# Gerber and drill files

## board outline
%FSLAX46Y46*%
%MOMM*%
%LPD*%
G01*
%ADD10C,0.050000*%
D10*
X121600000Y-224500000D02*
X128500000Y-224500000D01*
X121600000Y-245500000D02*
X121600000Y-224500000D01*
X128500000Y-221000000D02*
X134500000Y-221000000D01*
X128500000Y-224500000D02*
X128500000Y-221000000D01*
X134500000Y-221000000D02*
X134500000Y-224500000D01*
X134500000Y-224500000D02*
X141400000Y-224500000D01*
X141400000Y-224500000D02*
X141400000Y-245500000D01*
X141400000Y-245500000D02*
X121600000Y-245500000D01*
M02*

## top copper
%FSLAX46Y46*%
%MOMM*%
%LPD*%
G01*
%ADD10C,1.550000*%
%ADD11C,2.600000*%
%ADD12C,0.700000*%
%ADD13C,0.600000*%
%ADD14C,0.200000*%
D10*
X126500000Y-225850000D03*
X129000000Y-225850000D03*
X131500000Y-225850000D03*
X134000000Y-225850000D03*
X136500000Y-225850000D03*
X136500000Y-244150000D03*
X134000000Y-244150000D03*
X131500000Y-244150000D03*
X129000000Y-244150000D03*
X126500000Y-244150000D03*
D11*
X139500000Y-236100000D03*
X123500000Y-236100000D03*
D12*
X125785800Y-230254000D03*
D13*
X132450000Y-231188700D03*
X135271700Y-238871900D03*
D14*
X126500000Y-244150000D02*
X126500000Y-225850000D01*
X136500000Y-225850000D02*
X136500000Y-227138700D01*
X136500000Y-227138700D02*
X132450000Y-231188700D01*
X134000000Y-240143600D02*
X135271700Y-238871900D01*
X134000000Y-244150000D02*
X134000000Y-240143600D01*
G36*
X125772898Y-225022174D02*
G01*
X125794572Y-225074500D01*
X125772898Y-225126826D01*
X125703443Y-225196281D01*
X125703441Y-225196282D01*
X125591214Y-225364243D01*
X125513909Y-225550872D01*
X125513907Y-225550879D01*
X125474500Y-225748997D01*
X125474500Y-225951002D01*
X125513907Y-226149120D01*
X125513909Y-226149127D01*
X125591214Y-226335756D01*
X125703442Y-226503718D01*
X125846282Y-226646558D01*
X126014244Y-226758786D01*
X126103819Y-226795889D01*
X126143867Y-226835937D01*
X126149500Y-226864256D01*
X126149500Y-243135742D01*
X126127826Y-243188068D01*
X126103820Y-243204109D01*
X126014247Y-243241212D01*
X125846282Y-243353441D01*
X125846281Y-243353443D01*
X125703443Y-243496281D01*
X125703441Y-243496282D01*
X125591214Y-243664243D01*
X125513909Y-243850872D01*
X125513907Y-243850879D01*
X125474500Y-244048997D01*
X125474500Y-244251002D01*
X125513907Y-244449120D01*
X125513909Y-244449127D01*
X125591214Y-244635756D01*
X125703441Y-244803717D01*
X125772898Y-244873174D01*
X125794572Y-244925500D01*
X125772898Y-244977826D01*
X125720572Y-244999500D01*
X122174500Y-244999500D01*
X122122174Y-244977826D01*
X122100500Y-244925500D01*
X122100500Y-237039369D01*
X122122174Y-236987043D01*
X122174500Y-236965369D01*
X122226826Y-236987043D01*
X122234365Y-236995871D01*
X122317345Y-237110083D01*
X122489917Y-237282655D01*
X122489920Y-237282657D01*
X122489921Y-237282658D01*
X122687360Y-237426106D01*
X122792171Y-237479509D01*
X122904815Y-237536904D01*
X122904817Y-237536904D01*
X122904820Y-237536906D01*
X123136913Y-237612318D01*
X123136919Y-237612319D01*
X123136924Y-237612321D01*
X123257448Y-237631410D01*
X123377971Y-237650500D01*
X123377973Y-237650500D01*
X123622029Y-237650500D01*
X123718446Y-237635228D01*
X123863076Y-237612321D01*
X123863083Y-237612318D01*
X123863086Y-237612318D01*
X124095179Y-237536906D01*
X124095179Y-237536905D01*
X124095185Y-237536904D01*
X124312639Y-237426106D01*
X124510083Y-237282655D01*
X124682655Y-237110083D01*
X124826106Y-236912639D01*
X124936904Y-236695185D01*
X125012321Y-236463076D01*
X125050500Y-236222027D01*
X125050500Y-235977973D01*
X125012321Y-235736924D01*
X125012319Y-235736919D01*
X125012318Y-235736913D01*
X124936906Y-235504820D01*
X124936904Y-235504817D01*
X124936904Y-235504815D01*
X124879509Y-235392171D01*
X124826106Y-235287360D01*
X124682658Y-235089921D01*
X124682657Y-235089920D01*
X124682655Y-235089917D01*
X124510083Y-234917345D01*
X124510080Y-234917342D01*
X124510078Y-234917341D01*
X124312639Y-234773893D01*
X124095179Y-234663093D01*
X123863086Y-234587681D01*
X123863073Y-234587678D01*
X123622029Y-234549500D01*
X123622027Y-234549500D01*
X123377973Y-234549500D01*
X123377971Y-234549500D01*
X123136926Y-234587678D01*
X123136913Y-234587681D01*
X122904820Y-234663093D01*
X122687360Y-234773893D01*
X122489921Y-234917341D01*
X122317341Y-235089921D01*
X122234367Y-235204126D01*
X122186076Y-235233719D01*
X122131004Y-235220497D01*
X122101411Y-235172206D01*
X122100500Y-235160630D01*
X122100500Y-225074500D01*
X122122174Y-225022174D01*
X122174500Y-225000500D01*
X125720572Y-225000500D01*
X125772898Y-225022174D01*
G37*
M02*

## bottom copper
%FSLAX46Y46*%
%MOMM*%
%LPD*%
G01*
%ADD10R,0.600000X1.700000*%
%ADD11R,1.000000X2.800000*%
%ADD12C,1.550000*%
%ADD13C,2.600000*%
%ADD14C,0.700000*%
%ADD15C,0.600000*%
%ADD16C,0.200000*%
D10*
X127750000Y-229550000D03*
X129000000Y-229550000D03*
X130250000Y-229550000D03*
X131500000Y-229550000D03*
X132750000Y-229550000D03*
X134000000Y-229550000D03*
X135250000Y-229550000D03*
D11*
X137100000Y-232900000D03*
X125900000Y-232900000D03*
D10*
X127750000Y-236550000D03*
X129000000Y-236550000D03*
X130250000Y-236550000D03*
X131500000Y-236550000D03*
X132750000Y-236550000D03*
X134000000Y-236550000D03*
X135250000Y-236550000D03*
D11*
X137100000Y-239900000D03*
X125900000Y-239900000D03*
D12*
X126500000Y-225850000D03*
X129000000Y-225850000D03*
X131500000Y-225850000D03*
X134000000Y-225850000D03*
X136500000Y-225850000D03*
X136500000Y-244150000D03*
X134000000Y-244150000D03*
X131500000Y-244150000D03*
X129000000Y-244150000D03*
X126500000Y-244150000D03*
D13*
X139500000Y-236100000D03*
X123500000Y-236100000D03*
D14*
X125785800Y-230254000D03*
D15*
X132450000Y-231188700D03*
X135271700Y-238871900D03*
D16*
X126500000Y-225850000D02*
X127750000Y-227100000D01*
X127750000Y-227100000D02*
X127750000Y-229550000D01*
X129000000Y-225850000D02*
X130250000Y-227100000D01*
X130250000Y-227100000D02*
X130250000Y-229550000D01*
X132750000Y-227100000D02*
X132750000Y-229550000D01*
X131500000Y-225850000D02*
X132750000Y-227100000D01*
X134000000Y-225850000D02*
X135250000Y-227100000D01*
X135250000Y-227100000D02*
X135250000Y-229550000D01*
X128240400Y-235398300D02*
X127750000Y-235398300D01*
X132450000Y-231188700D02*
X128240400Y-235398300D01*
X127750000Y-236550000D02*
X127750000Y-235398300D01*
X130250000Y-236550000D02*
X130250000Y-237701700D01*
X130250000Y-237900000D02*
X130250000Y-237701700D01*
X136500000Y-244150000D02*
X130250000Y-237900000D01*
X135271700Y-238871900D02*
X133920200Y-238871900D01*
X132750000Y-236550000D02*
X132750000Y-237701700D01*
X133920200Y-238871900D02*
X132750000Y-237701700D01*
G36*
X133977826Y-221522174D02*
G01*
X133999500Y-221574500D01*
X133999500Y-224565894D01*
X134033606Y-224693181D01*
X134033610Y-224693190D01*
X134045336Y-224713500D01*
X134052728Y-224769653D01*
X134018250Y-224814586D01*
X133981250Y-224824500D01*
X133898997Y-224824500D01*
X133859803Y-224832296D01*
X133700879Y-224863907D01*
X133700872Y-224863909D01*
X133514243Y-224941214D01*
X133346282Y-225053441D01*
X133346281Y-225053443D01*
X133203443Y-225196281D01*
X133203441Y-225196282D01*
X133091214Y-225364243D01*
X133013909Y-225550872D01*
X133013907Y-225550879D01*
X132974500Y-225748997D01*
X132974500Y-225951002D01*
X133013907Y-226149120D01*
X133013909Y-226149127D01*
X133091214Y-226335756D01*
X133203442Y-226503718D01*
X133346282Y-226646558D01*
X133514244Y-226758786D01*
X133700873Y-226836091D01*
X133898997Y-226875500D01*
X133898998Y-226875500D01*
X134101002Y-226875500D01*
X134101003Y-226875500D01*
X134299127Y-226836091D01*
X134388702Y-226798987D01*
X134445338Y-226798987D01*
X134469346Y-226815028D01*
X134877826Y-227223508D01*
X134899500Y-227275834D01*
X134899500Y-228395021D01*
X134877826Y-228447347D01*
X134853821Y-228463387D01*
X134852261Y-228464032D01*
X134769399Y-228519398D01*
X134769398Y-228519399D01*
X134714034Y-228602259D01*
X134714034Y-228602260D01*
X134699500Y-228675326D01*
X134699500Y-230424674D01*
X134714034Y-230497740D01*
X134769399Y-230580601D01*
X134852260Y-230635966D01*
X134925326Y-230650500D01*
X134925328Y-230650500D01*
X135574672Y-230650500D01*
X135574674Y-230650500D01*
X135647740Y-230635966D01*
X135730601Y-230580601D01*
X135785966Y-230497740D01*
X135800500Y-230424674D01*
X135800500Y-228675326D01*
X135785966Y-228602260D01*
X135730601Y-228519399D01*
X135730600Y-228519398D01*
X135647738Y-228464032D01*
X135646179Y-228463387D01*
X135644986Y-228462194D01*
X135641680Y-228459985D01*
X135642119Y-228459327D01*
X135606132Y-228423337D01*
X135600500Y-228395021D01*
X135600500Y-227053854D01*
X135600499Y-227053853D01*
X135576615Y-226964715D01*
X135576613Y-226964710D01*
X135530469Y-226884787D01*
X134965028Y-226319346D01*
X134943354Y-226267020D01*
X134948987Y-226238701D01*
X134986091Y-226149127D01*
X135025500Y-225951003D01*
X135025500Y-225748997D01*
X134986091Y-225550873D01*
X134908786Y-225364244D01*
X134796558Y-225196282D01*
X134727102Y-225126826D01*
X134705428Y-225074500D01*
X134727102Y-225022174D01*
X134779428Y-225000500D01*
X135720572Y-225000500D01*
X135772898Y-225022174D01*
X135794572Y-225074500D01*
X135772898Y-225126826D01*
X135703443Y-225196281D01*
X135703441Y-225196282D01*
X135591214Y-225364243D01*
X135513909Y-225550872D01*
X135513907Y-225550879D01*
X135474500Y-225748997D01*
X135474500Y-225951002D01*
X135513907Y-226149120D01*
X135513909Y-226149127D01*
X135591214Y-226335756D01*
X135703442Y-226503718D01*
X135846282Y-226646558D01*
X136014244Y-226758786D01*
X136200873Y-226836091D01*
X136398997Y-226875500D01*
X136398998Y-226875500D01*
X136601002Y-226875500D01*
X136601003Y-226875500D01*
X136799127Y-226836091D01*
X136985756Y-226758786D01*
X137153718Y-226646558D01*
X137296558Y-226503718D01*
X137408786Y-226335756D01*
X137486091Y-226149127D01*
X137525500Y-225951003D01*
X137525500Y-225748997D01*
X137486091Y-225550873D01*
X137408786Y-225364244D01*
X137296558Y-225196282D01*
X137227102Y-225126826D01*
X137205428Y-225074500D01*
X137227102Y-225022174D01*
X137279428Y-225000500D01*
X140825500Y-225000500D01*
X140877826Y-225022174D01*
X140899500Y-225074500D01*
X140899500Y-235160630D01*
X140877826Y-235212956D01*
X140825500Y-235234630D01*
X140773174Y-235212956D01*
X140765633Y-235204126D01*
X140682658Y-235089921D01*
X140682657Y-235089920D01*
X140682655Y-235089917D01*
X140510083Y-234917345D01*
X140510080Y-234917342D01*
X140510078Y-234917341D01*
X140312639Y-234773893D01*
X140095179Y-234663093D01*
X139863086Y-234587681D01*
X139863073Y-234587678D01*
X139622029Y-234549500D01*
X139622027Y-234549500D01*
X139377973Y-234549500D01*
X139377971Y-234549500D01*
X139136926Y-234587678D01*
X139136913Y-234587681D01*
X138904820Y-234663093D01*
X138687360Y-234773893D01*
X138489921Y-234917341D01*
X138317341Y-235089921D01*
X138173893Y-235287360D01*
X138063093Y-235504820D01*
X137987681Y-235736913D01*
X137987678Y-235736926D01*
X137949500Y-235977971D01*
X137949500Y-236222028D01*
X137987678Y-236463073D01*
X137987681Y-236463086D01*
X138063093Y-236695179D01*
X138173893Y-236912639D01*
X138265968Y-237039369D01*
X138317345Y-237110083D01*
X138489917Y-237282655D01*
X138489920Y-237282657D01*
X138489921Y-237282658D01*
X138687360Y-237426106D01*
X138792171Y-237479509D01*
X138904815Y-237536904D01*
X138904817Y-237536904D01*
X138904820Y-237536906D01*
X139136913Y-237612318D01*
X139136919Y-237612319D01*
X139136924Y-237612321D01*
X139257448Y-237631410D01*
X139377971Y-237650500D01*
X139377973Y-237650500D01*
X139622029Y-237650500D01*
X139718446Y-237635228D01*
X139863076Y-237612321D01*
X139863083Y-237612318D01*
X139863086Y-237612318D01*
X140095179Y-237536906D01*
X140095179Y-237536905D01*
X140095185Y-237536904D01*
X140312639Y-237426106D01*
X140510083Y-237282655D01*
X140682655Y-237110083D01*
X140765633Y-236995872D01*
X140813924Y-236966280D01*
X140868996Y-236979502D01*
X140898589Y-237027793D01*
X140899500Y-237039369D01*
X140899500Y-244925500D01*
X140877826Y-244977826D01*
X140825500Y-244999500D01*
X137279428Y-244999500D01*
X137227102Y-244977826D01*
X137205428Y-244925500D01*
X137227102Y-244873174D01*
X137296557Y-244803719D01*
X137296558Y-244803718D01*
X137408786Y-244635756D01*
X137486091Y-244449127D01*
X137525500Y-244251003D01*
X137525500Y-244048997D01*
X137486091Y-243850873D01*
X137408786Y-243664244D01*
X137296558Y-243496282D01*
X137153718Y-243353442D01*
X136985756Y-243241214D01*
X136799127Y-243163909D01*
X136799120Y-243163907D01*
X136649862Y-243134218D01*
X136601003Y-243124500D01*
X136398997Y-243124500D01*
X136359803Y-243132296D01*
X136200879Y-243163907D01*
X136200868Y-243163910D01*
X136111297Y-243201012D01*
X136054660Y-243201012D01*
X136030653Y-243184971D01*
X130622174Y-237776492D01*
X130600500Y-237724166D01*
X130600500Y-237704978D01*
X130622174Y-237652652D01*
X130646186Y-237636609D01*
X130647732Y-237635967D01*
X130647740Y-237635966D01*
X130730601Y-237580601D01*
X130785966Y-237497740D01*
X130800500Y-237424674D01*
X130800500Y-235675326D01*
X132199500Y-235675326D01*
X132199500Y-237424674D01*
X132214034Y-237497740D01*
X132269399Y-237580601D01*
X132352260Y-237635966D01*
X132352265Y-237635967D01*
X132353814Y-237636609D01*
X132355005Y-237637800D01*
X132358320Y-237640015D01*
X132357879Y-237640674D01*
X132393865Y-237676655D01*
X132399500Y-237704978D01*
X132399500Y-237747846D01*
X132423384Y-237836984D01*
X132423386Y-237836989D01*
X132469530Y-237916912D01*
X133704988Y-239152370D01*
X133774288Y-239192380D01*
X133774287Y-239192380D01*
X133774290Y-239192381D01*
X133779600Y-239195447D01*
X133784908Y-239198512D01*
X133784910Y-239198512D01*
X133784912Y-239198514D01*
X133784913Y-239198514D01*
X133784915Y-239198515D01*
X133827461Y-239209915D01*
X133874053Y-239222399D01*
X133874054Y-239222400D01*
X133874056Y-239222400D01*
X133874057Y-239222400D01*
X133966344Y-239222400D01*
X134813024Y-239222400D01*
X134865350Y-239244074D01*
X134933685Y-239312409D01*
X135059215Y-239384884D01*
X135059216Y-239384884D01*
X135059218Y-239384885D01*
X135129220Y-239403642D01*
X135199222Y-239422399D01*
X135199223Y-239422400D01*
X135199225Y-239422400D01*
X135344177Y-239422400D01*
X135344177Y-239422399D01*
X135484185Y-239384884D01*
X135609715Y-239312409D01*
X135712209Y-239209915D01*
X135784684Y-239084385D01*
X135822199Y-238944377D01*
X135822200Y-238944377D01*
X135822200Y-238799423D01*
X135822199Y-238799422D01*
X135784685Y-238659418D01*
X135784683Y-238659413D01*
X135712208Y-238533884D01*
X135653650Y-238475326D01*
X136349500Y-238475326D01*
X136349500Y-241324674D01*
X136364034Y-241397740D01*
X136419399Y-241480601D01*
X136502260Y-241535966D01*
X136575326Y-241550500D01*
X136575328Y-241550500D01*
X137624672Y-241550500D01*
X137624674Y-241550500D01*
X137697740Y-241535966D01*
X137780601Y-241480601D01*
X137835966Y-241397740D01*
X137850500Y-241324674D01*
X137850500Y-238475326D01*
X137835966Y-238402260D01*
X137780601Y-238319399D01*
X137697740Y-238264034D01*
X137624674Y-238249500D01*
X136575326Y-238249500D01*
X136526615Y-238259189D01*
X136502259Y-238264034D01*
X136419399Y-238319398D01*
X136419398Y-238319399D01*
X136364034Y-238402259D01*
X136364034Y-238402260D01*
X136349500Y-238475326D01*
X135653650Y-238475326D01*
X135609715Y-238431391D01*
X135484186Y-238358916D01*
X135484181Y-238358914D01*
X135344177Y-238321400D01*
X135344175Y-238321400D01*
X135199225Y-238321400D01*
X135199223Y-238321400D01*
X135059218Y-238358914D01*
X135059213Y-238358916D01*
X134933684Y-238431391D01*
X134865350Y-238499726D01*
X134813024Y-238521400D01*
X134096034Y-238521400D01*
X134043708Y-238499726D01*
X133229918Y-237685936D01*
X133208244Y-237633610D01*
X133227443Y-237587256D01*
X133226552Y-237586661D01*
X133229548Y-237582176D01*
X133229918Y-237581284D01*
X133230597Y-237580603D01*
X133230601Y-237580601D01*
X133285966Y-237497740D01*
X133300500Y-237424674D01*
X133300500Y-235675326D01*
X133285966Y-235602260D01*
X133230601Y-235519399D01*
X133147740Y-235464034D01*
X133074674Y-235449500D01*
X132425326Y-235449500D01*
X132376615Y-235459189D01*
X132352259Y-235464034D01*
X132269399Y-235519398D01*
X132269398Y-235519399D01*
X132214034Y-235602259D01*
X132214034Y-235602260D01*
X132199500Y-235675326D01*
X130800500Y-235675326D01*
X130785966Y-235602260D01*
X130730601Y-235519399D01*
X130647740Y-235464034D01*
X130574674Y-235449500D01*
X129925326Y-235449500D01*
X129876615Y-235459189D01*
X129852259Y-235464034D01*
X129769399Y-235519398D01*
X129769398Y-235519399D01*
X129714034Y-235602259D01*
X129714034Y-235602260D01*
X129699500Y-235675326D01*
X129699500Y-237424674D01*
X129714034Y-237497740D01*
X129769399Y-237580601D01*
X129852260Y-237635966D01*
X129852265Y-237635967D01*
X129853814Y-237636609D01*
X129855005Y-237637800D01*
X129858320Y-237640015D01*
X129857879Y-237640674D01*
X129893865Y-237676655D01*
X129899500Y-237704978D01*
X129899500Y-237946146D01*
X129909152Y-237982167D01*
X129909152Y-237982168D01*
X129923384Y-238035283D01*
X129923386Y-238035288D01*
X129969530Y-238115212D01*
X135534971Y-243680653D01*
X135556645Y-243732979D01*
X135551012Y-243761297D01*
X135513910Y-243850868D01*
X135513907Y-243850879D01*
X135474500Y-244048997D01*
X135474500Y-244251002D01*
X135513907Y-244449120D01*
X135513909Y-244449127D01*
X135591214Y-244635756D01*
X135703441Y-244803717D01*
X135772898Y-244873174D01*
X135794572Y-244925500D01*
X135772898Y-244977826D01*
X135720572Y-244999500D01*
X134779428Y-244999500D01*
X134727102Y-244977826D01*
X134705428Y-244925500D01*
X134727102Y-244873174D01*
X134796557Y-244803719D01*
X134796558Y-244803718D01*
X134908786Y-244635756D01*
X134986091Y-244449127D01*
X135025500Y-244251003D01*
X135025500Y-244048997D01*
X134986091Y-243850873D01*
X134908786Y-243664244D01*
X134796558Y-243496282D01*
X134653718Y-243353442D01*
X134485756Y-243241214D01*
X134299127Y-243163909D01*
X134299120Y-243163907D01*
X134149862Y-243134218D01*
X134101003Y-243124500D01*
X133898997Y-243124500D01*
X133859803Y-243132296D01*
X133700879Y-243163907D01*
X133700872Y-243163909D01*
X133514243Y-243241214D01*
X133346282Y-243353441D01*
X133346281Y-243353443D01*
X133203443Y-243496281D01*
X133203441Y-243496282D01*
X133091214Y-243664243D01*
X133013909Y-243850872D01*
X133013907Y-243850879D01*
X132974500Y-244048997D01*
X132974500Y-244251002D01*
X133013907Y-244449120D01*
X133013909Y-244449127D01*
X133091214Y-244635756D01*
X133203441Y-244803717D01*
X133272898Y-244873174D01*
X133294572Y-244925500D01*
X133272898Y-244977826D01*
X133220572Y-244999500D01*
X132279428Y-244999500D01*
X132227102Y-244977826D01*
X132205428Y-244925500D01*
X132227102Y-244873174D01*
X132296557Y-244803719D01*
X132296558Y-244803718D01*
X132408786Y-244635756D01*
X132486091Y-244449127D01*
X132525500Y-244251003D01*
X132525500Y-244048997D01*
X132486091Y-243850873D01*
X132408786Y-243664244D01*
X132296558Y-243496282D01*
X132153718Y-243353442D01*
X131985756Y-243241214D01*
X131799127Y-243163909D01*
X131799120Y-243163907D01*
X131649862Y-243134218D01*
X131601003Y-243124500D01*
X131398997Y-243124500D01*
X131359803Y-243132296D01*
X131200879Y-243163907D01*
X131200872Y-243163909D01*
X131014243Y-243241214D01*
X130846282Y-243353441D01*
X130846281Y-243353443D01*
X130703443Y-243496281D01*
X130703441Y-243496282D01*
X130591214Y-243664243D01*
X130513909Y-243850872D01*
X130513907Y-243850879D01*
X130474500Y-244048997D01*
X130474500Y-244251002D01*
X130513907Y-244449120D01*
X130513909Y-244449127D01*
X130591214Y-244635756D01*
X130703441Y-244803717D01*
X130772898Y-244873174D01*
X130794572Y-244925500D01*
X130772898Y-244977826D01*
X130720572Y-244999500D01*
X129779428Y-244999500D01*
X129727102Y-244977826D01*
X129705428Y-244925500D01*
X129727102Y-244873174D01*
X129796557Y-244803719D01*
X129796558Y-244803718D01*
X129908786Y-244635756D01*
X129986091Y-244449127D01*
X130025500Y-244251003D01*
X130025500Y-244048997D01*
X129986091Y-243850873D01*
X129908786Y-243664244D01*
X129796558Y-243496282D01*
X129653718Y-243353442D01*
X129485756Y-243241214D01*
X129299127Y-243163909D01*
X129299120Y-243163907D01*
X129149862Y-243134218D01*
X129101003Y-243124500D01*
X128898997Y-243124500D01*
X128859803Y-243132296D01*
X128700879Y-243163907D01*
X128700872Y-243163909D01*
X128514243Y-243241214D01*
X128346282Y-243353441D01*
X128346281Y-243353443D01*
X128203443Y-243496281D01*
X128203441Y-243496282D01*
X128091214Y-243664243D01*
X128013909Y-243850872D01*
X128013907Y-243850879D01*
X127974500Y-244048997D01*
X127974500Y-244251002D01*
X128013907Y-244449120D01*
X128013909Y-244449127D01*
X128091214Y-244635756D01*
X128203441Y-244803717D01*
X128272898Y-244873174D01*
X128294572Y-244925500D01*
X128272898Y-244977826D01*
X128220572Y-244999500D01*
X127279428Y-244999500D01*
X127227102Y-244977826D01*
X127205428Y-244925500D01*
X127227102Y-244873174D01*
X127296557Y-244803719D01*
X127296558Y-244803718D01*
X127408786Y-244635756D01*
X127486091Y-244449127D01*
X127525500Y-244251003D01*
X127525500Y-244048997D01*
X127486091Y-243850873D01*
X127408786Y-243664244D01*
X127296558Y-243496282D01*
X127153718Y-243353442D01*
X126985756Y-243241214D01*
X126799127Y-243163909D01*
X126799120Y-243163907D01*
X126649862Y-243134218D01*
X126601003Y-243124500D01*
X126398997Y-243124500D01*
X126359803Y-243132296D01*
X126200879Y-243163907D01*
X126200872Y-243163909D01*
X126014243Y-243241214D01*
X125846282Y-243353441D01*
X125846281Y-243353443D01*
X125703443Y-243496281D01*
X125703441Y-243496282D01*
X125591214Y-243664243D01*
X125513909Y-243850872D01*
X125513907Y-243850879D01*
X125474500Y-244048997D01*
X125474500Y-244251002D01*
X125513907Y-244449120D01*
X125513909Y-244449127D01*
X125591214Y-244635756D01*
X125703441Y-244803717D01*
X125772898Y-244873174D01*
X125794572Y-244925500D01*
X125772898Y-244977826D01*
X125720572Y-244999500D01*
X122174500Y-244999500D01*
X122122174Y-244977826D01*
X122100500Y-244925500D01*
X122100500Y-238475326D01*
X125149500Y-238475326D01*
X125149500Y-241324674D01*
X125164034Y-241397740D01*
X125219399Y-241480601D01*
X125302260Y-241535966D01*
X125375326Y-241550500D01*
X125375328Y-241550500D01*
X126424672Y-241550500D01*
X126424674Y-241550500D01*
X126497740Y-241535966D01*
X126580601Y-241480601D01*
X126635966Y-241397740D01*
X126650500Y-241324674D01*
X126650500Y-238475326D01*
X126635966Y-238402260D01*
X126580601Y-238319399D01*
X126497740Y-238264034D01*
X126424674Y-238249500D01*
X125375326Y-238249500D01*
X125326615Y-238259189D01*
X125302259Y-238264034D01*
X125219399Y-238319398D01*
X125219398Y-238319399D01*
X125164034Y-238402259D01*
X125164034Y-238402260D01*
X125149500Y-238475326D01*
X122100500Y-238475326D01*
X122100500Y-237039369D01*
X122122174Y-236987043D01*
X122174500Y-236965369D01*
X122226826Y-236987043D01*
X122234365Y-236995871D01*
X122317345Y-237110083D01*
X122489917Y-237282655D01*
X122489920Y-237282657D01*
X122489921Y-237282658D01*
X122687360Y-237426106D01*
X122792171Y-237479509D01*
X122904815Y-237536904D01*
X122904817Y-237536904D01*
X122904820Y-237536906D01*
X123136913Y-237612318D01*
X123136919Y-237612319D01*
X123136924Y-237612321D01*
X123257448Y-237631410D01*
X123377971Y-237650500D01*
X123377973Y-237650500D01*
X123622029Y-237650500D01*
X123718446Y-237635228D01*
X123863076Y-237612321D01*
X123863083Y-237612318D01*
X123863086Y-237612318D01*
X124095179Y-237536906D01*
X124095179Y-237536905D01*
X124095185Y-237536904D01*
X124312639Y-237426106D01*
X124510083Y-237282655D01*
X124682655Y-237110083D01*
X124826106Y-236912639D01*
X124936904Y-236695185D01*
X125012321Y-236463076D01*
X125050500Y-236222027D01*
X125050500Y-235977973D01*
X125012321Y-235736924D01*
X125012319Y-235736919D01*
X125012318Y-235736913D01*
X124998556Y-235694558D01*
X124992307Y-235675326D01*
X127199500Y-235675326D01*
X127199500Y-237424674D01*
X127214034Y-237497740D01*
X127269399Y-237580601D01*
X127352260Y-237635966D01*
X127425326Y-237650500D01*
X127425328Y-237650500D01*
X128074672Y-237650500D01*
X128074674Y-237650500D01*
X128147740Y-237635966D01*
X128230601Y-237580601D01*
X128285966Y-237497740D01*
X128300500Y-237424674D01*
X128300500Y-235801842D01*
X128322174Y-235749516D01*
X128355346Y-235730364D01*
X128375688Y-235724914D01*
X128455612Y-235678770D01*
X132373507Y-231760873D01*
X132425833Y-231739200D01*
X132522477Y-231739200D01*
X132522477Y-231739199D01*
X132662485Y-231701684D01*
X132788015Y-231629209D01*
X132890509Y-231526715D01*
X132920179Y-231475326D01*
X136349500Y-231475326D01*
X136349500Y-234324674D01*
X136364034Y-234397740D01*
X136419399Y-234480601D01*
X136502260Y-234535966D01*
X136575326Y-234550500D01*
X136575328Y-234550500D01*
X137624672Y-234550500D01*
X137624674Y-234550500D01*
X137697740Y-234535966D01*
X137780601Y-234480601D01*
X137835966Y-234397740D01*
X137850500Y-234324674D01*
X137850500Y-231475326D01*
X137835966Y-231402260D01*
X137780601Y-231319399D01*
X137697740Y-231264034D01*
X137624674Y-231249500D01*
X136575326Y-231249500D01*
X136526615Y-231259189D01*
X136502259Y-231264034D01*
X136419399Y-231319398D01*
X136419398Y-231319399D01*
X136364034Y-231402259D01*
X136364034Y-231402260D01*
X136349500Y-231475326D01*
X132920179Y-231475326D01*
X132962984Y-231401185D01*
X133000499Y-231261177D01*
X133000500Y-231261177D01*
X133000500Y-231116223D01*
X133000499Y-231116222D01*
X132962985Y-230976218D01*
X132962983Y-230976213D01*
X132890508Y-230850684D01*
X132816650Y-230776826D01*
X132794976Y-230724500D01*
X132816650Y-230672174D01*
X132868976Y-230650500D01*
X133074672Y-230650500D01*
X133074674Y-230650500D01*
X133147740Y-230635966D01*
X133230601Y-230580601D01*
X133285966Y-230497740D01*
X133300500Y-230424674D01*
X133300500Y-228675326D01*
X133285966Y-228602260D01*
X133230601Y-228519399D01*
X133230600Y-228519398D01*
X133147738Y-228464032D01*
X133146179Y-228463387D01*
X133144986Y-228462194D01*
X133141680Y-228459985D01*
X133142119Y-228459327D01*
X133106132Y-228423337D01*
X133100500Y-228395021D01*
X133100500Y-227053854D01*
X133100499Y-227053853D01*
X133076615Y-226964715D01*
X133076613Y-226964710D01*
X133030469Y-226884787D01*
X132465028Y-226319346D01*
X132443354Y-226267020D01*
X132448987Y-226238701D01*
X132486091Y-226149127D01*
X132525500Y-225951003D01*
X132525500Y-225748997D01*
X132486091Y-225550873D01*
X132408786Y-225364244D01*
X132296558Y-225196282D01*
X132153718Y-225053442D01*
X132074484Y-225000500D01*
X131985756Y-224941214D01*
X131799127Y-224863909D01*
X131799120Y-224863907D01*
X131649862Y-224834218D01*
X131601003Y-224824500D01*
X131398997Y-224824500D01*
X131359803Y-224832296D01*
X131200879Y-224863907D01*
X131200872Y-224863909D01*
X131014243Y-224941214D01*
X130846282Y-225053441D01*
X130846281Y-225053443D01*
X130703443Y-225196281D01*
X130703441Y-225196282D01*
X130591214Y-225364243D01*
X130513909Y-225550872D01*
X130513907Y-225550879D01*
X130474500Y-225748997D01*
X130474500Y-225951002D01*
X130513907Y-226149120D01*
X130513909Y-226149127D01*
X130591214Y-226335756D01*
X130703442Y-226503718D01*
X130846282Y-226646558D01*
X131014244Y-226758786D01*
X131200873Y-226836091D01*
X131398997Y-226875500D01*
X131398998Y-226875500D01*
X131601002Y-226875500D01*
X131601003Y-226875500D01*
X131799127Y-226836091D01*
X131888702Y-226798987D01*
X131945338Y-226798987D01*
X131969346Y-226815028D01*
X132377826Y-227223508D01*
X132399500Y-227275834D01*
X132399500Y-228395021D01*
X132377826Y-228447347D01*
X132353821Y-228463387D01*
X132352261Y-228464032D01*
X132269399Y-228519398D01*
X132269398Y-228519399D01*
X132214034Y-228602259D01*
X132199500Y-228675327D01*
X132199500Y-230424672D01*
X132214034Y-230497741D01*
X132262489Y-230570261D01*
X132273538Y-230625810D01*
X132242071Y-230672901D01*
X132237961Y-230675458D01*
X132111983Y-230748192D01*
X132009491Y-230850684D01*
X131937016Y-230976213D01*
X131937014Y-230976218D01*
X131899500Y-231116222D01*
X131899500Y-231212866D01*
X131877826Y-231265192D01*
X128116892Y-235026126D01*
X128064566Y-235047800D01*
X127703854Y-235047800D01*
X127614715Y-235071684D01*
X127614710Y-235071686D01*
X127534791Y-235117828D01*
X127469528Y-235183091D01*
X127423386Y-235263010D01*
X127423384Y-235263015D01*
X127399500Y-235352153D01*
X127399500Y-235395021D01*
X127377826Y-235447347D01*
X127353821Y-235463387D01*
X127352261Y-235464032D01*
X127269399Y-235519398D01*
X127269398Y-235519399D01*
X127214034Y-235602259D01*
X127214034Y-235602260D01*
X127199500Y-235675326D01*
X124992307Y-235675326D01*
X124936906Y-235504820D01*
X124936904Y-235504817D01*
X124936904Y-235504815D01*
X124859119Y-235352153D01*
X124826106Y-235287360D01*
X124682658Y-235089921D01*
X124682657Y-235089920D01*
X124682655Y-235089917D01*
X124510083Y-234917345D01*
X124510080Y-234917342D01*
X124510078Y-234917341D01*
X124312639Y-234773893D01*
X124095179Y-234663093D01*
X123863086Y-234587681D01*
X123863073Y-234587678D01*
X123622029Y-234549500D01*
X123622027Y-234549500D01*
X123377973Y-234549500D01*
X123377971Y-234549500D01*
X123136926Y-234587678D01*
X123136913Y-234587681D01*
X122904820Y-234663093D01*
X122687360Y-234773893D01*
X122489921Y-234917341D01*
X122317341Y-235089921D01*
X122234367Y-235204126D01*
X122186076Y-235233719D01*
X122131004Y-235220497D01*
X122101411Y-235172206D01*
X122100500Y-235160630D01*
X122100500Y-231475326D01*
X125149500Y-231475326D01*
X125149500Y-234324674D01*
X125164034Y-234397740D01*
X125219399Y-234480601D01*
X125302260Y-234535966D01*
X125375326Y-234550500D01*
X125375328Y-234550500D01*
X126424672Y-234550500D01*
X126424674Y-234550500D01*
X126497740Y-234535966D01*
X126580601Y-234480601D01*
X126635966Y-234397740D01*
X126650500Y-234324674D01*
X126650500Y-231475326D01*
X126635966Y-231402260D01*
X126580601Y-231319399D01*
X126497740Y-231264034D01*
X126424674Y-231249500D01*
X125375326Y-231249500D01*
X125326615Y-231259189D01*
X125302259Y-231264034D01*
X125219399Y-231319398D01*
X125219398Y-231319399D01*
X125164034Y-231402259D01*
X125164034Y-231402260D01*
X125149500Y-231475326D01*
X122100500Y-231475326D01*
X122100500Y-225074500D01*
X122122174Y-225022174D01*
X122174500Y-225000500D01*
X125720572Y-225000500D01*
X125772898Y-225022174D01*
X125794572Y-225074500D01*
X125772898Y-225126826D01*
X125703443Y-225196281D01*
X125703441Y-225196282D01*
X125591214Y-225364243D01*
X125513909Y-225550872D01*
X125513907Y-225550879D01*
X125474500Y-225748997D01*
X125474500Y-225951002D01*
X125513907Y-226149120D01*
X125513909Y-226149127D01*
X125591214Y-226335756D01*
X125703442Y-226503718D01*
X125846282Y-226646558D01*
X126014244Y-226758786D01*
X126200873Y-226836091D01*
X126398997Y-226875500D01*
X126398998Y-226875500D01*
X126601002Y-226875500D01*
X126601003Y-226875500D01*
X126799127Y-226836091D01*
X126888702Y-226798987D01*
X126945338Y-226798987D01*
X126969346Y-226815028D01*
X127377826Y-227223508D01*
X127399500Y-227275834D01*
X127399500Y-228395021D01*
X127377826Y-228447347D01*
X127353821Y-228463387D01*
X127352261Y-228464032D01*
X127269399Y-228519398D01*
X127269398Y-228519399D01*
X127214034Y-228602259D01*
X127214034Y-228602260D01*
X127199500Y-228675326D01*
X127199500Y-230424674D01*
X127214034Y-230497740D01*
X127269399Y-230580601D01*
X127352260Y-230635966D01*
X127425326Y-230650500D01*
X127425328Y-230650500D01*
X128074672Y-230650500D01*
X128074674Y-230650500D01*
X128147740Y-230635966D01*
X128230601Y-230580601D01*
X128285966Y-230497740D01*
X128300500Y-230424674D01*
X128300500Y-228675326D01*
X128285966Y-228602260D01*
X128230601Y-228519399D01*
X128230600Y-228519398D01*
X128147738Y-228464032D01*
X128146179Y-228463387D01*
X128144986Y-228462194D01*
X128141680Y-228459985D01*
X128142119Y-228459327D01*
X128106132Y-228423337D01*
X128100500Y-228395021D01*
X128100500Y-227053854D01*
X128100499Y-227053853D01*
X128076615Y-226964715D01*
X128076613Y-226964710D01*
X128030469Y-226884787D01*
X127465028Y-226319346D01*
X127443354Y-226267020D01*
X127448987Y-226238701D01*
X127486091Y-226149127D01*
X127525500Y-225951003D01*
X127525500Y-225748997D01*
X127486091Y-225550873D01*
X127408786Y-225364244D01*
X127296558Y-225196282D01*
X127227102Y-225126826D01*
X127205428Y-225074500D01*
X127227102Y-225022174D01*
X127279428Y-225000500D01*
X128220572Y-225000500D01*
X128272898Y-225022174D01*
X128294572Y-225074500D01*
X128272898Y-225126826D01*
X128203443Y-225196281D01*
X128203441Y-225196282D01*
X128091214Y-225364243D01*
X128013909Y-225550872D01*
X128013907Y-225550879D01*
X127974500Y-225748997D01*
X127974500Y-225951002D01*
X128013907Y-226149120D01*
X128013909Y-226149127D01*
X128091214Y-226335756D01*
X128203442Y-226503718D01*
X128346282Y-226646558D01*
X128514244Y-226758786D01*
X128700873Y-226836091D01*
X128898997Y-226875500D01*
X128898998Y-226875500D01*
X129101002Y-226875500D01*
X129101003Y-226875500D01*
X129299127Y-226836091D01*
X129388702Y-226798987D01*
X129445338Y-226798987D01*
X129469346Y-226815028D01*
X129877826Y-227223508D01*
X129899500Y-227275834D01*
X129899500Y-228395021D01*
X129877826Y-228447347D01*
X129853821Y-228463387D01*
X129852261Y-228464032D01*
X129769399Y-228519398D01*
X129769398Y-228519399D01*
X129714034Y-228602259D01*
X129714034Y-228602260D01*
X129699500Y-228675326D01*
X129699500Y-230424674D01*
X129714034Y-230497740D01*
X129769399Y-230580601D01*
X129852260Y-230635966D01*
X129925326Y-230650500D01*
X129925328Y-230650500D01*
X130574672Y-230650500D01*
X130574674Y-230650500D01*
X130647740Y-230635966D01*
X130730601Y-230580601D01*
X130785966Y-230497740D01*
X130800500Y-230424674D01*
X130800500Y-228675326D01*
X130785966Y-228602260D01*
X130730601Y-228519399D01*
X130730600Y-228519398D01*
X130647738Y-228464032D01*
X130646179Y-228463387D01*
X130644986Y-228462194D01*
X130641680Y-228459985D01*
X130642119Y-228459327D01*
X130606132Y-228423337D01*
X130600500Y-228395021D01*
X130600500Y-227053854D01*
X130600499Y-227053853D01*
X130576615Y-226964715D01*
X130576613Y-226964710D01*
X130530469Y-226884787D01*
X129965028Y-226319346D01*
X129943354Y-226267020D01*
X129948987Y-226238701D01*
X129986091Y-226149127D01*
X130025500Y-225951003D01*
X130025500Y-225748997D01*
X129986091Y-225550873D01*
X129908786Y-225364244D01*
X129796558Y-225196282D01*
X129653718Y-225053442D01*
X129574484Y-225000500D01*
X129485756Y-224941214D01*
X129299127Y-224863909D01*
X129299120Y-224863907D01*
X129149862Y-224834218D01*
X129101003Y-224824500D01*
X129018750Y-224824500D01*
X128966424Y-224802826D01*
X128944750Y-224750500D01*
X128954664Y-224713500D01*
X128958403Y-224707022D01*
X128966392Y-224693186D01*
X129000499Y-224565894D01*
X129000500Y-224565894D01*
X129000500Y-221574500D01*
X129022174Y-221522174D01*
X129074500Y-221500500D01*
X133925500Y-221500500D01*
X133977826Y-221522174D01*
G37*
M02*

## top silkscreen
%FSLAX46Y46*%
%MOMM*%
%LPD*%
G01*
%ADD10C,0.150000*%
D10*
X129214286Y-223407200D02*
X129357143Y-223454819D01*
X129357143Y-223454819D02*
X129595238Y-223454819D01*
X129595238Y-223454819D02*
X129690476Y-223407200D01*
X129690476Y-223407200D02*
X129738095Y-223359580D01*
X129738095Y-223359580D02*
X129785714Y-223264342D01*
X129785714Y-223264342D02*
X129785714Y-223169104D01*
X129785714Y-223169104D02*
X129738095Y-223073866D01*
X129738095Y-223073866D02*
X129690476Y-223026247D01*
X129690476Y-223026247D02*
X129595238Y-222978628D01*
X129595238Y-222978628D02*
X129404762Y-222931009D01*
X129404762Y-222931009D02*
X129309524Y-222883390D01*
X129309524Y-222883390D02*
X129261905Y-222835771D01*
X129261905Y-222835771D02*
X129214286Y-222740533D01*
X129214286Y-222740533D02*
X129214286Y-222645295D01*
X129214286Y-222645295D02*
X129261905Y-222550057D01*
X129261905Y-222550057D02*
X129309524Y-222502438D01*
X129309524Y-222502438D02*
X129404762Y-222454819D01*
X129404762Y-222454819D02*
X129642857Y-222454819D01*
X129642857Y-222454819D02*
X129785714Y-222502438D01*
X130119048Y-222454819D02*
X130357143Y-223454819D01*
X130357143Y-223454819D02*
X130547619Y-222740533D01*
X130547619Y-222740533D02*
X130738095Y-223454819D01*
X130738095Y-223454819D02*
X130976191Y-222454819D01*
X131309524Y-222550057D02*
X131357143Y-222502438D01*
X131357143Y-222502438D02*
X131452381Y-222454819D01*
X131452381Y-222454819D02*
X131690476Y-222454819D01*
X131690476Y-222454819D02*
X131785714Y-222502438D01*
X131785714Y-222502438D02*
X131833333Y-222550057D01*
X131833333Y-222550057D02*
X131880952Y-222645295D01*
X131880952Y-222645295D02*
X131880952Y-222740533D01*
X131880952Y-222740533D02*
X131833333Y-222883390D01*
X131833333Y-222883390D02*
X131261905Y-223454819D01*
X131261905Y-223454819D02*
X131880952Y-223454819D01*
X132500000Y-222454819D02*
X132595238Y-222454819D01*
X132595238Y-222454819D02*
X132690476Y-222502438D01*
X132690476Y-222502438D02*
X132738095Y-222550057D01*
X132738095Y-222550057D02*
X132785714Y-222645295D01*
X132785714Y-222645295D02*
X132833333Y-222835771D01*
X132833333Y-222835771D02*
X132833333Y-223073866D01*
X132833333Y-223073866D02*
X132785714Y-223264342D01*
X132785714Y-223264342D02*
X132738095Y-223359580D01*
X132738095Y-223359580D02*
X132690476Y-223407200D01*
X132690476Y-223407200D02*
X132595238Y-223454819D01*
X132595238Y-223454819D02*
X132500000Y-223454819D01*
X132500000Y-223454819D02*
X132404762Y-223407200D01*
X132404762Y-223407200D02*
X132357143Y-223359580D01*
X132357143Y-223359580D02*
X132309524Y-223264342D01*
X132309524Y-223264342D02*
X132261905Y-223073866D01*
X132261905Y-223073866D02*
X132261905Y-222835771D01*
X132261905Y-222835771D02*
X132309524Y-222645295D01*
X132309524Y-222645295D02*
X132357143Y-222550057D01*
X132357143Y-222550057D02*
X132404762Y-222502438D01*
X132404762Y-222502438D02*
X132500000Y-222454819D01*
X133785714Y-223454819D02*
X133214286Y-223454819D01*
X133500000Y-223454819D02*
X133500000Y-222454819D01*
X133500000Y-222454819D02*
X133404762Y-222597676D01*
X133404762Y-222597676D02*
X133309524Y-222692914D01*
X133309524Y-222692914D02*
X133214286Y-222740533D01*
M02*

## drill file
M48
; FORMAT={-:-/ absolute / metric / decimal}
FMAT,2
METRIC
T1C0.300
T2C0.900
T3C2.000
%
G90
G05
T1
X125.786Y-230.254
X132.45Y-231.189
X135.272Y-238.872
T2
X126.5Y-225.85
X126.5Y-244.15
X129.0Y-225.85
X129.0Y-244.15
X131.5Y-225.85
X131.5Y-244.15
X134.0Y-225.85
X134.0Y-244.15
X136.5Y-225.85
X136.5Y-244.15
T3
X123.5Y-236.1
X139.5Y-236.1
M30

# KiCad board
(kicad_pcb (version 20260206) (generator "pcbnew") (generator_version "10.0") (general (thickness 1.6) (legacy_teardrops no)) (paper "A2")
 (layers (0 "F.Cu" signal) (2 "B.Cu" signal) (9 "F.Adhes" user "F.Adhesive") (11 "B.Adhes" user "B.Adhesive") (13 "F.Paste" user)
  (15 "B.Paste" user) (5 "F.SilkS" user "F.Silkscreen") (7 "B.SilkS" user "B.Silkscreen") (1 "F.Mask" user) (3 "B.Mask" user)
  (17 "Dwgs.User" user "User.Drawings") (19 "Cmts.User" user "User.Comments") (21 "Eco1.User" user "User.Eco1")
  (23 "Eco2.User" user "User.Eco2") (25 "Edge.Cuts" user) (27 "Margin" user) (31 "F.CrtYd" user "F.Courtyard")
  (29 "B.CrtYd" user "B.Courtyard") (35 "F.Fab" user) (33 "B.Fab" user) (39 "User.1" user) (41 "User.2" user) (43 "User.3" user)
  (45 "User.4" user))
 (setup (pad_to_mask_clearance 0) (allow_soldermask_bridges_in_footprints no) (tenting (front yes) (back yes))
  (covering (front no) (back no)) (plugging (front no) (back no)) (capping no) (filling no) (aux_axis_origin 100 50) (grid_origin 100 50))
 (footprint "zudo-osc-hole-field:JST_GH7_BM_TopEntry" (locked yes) (layer "B.Cu") (at 131.5 229.55 180)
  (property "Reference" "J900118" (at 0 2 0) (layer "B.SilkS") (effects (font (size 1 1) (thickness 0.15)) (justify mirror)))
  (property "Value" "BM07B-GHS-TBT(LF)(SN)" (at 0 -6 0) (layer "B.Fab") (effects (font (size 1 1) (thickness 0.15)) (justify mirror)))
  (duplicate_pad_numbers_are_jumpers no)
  (pad "1" smd rect (at 3.75 0 180) (size 0.6 1.7) (layers "B.Cu" "B.Mask" "B.Paste") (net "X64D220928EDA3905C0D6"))
  (pad "2" smd rect (at 2.5 0 180) (size 0.6 1.7) (layers "B.Cu" "B.Mask" "B.Paste") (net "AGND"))
  (pad "3" smd rect (at 1.25 0 180) (size 0.6 1.7) (layers "B.Cu" "B.Mask" "B.Paste") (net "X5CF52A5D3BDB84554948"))
  (pad "4" smd rect (at 0 0 180) (size 0.6 1.7) (layers "B.Cu" "B.Mask" "B.Paste") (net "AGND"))
  (pad "5" smd rect (at -1.25 0 180) (size 0.6 1.7) (layers "B.Cu" "B.Mask" "B.Paste") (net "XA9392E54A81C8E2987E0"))
  (pad "6" smd rect (at -2.5 0 180) (size 0.6 1.7) (layers "B.Cu" "B.Mask" "B.Paste") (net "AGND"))
  (pad "7" smd rect (at -3.75 0 180) (size 0.6 1.7) (layers "B.Cu" "B.Mask" "B.Paste") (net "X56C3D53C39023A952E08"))
  (pad "MP1" smd rect (at -5.6 -3.35 180) (size 1 2.8) (layers "B.Cu" "B.Mask" "B.Paste") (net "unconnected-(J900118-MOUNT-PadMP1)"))
  (pad "MP2" smd rect (at 5.6 -3.35 180) (size 1 2.8) (layers "B.Cu" "B.Mask" "B.Paste") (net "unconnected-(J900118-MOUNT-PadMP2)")))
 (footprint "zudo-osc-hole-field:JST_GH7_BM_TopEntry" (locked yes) (layer "B.Cu") (at 131.5 236.55 180)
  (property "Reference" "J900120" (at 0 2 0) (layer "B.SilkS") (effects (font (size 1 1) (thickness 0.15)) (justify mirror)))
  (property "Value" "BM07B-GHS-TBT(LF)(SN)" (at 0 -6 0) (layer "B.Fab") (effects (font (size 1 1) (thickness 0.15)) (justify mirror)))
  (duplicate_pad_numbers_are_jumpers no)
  (pad "1" smd rect (at 3.75 0 180) (size 0.6 1.7) (layers "B.Cu" "B.Mask" "B.Paste") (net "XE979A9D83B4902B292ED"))
  (pad "2" smd rect (at 2.5 0 180) (size 0.6 1.7) (layers "B.Cu" "B.Mask" "B.Paste") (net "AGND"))
  (pad "3" smd rect (at 1.25 0 180) (size 0.6 1.7) (layers "B.Cu" "B.Mask" "B.Paste") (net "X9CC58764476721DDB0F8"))
  (pad "4" smd rect (at 0 0 180) (size 0.6 1.7) (layers "B.Cu" "B.Mask" "B.Paste") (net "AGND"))
  (pad "5" smd rect (at -1.25 0 180) (size 0.6 1.7) (layers "B.Cu" "B.Mask" "B.Paste") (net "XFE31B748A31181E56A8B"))
  (pad "6" smd rect (at -2.5 0 180) (size 0.6 1.7) (layers "B.Cu" "B.Mask" "B.Paste") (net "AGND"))
  (pad "7" smd rect (at -3.75 0 180) (size 0.6 1.7) (layers "B.Cu" "B.Mask" "B.Paste") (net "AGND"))
  (pad "MP1" smd rect (at -5.6 -3.35 180) (size 1 2.8) (layers "B.Cu" "B.Mask" "B.Paste") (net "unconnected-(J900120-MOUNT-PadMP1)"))
  (pad "MP2" smd rect (at 5.6 -3.35 180) (size 1 2.8) (layers "B.Cu" "B.Mask" "B.Paste") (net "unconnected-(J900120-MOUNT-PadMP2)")))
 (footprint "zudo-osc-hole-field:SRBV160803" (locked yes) (layer "F.Cu") (at 131.5 235 180)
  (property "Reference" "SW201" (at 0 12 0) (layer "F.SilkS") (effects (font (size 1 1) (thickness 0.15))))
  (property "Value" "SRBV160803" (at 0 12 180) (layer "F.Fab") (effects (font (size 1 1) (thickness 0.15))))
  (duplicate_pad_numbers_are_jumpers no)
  (pad "1" thru_hole circle (at 5 9.15 180) (size 1.55 1.55) (drill 0.9) (layers "*.Cu" "*.Mask") (remove_unused_layers no)
   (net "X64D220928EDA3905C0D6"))
  (pad "2" thru_hole circle (at 2.5 9.15 180) (size 1.55 1.55) (drill 0.9) (layers "*.Cu" "*.Mask") (remove_unused_layers no)
   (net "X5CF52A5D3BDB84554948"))
  (pad "3" thru_hole circle (at 0 9.15 180) (size 1.55 1.55) (drill 0.9) (layers "*.Cu" "*.Mask") (remove_unused_layers no)
   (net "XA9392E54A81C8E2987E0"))
  (pad "4" thru_hole circle (at -2.5 9.15 180) (size 1.55 1.55) (drill 0.9) (layers "*.Cu" "*.Mask") (remove_unused_layers no)
   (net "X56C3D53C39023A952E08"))
  (pad "5" thru_hole circle (at -5 9.15 180) (size 1.55 1.55) (drill 0.9) (layers "*.Cu" "*.Mask") (remove_unused_layers no)
   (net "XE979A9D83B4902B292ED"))
  (pad "6" thru_hole circle (at -5 -9.15 180) (size 1.55 1.55) (drill 0.9) (layers "*.Cu" "*.Mask") (remove_unused_layers no)
   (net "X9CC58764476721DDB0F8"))
  (pad "7" thru_hole circle (at -2.5 -9.15 180) (size 1.55 1.55) (drill 0.9) (layers "*.Cu" "*.Mask") (remove_unused_layers no)
   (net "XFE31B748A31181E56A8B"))
  (pad "8" thru_hole circle (at 0 -9.15 180) (size 1.55 1.55) (drill 0.9) (layers "*.Cu" "*.Mask") (remove_unused_layers no)
   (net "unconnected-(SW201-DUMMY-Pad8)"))
  (pad "9" thru_hole circle (at 2.5 -9.15 180) (size 1.55 1.55) (drill 0.9) (layers "*.Cu" "*.Mask") (remove_unused_layers no)
   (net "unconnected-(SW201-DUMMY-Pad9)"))
  (pad "10" thru_hole circle (at 5 -9.15 180) (size 1.55 1.55) (drill 0.9) (layers "*.Cu" "*.Mask") (remove_unused_layers no)
   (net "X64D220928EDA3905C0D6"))
  (pad "MP1" thru_hole circle (at -8 -1.1 180) (size 2.6 2.6) (drill 2) (layers "*.Cu" "*.Mask") (remove_unused_layers no)
   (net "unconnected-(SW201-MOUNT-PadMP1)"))
  (pad "MP2" thru_hole circle (at 8 -1.1 180) (size 2.6 2.6) (drill 2) (layers "*.Cu" "*.Mask") (remove_unused_layers no)
   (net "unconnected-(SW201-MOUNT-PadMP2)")))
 (gr_line (start 121.6 224.5) (end 128.5 224.5) (stroke (width 0.05) (type default)) (layer "Edge.Cuts"))
 (gr_line (start 121.6 245.5) (end 121.6 224.5) (stroke (width 0.05) (type default)) (layer "Edge.Cuts"))
 (gr_line (start 128.5 221) (end 134.5 221) (stroke (width 0.05) (type default)) (layer "Edge.Cuts"))
 (gr_line (start 128.5 224.5) (end 128.5 221) (stroke (width 0.05) (type default)) (layer "Edge.Cuts"))
 (gr_line (start 134.5 221) (end 134.5 224.5) (stroke (width 0.05) (type default)) (layer "Edge.Cuts"))
 (gr_line (start 134.5 224.5) (end 141.4 224.5) (stroke (width 0.05) (type default)) (layer "Edge.Cuts"))
 (gr_line (start 141.4 224.5) (end 141.4 245.5) (stroke (width 0.05) (type default)) (layer "Edge.Cuts"))
 (gr_line (start 141.4 245.5) (end 121.6 245.5) (stroke (width 0.05) (type default)) (layer "Edge.Cuts"))
 (segment (start 126.5 244.15) (end 126.5 225.85) (width 0.2) (layer "F.Cu") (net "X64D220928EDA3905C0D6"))
 (segment (start 126.5 225.85) (end 127.75 227.1) (width 0.2) (layer "B.Cu") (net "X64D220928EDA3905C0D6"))
 (segment (start 127.75 227.1) (end 127.75 229.55) (width 0.2) (layer "B.Cu") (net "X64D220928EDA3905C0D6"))
 (via (at 125.7858 230.254) (size 0.7) (drill 0.3) (layers "F.Cu" "B.Cu") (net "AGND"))
 (segment (start 129 225.85) (end 130.25 227.1) (width 0.2) (layer "B.Cu") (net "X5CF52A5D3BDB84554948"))
 (segment (start 130.25 227.1) (end 130.25 229.55) (width 0.2) (layer "B.Cu") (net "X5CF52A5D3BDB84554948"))
 (segment (start 132.75 227.1) (end 132.75 229.55) (width 0.2) (layer "B.Cu") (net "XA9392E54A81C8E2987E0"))
 (segment (start 131.5 225.85) (end 132.75 227.1) (width 0.2) (layer "B.Cu") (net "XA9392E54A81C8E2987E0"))
 (segment (start 134 225.85) (end 135.25 227.1) (width 0.2) (layer "B.Cu") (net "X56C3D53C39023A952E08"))
 (segment (start 135.25 227.1) (end 135.25 229.55) (width 0.2) (layer "B.Cu") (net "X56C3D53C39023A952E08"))
 (segment (start 136.5 225.85) (end 136.5 227.1387) (width 0.2) (layer "F.Cu") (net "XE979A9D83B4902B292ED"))
 (segment (start 136.5 227.1387) (end 132.45 231.1887) (width 0.2) (layer "F.Cu") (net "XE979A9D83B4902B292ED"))
 (via (at 132.45 231.1887) (size 0.6) (drill 0.3) (layers "F.Cu" "B.Cu") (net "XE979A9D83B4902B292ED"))
 (segment (start 128.2404 235.3983) (end 127.75 235.3983) (width 0.2) (layer "B.Cu") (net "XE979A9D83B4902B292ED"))
 (segment (start 132.45 231.1887) (end 128.2404 235.3983) (width 0.2) (layer "B.Cu") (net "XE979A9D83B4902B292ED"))
 (segment (start 127.75 236.55) (end 127.75 235.3983) (width 0.2) (layer "B.Cu") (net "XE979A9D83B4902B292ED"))
 (segment (start 130.25 236.55) (end 130.25 237.7017) (width 0.2) (layer "B.Cu") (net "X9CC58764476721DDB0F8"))
 (segment (start 130.25 237.9) (end 130.25 237.7017) (width 0.2) (layer "B.Cu") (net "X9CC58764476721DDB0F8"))
 (segment (start 136.5 244.15) (end 130.25 237.9) (width 0.2) (layer "B.Cu") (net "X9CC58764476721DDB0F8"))
 (segment (start 134 240.1436) (end 135.2717 238.8719) (width 0.2) (layer "F.Cu") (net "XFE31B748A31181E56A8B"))
 (segment (start 134 244.15) (end 134 240.1436) (width 0.2) (layer "F.Cu") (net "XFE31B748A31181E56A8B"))
 (via (at 135.2717 238.8719) (size 0.6) (drill 0.3) (layers "F.Cu" "B.Cu") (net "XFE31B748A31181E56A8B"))
 (segment (start 135.2717 238.8719) (end 133.9202 238.8719) (width 0.2) (layer "B.Cu") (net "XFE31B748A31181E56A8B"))
 (segment (start 132.75 236.55) (end 132.75 237.7017) (width 0.2) (layer "B.Cu") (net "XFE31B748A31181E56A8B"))
 (segment (start 133.9202 238.8719) (end 132.75 237.7017) (width 0.2) (layer "B.Cu") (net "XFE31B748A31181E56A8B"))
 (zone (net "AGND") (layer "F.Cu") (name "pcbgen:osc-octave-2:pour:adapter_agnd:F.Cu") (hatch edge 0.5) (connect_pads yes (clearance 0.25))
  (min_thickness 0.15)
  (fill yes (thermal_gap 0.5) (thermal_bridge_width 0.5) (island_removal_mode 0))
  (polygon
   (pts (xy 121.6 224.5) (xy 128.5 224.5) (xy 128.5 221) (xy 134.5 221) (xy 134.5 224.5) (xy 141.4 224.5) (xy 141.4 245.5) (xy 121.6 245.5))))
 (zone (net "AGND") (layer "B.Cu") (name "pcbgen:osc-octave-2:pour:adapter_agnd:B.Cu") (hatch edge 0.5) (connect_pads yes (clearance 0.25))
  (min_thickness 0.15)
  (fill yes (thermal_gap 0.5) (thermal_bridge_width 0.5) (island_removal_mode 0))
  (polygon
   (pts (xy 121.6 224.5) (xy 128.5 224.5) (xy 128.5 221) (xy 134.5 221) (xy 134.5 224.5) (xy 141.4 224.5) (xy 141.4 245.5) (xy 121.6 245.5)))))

